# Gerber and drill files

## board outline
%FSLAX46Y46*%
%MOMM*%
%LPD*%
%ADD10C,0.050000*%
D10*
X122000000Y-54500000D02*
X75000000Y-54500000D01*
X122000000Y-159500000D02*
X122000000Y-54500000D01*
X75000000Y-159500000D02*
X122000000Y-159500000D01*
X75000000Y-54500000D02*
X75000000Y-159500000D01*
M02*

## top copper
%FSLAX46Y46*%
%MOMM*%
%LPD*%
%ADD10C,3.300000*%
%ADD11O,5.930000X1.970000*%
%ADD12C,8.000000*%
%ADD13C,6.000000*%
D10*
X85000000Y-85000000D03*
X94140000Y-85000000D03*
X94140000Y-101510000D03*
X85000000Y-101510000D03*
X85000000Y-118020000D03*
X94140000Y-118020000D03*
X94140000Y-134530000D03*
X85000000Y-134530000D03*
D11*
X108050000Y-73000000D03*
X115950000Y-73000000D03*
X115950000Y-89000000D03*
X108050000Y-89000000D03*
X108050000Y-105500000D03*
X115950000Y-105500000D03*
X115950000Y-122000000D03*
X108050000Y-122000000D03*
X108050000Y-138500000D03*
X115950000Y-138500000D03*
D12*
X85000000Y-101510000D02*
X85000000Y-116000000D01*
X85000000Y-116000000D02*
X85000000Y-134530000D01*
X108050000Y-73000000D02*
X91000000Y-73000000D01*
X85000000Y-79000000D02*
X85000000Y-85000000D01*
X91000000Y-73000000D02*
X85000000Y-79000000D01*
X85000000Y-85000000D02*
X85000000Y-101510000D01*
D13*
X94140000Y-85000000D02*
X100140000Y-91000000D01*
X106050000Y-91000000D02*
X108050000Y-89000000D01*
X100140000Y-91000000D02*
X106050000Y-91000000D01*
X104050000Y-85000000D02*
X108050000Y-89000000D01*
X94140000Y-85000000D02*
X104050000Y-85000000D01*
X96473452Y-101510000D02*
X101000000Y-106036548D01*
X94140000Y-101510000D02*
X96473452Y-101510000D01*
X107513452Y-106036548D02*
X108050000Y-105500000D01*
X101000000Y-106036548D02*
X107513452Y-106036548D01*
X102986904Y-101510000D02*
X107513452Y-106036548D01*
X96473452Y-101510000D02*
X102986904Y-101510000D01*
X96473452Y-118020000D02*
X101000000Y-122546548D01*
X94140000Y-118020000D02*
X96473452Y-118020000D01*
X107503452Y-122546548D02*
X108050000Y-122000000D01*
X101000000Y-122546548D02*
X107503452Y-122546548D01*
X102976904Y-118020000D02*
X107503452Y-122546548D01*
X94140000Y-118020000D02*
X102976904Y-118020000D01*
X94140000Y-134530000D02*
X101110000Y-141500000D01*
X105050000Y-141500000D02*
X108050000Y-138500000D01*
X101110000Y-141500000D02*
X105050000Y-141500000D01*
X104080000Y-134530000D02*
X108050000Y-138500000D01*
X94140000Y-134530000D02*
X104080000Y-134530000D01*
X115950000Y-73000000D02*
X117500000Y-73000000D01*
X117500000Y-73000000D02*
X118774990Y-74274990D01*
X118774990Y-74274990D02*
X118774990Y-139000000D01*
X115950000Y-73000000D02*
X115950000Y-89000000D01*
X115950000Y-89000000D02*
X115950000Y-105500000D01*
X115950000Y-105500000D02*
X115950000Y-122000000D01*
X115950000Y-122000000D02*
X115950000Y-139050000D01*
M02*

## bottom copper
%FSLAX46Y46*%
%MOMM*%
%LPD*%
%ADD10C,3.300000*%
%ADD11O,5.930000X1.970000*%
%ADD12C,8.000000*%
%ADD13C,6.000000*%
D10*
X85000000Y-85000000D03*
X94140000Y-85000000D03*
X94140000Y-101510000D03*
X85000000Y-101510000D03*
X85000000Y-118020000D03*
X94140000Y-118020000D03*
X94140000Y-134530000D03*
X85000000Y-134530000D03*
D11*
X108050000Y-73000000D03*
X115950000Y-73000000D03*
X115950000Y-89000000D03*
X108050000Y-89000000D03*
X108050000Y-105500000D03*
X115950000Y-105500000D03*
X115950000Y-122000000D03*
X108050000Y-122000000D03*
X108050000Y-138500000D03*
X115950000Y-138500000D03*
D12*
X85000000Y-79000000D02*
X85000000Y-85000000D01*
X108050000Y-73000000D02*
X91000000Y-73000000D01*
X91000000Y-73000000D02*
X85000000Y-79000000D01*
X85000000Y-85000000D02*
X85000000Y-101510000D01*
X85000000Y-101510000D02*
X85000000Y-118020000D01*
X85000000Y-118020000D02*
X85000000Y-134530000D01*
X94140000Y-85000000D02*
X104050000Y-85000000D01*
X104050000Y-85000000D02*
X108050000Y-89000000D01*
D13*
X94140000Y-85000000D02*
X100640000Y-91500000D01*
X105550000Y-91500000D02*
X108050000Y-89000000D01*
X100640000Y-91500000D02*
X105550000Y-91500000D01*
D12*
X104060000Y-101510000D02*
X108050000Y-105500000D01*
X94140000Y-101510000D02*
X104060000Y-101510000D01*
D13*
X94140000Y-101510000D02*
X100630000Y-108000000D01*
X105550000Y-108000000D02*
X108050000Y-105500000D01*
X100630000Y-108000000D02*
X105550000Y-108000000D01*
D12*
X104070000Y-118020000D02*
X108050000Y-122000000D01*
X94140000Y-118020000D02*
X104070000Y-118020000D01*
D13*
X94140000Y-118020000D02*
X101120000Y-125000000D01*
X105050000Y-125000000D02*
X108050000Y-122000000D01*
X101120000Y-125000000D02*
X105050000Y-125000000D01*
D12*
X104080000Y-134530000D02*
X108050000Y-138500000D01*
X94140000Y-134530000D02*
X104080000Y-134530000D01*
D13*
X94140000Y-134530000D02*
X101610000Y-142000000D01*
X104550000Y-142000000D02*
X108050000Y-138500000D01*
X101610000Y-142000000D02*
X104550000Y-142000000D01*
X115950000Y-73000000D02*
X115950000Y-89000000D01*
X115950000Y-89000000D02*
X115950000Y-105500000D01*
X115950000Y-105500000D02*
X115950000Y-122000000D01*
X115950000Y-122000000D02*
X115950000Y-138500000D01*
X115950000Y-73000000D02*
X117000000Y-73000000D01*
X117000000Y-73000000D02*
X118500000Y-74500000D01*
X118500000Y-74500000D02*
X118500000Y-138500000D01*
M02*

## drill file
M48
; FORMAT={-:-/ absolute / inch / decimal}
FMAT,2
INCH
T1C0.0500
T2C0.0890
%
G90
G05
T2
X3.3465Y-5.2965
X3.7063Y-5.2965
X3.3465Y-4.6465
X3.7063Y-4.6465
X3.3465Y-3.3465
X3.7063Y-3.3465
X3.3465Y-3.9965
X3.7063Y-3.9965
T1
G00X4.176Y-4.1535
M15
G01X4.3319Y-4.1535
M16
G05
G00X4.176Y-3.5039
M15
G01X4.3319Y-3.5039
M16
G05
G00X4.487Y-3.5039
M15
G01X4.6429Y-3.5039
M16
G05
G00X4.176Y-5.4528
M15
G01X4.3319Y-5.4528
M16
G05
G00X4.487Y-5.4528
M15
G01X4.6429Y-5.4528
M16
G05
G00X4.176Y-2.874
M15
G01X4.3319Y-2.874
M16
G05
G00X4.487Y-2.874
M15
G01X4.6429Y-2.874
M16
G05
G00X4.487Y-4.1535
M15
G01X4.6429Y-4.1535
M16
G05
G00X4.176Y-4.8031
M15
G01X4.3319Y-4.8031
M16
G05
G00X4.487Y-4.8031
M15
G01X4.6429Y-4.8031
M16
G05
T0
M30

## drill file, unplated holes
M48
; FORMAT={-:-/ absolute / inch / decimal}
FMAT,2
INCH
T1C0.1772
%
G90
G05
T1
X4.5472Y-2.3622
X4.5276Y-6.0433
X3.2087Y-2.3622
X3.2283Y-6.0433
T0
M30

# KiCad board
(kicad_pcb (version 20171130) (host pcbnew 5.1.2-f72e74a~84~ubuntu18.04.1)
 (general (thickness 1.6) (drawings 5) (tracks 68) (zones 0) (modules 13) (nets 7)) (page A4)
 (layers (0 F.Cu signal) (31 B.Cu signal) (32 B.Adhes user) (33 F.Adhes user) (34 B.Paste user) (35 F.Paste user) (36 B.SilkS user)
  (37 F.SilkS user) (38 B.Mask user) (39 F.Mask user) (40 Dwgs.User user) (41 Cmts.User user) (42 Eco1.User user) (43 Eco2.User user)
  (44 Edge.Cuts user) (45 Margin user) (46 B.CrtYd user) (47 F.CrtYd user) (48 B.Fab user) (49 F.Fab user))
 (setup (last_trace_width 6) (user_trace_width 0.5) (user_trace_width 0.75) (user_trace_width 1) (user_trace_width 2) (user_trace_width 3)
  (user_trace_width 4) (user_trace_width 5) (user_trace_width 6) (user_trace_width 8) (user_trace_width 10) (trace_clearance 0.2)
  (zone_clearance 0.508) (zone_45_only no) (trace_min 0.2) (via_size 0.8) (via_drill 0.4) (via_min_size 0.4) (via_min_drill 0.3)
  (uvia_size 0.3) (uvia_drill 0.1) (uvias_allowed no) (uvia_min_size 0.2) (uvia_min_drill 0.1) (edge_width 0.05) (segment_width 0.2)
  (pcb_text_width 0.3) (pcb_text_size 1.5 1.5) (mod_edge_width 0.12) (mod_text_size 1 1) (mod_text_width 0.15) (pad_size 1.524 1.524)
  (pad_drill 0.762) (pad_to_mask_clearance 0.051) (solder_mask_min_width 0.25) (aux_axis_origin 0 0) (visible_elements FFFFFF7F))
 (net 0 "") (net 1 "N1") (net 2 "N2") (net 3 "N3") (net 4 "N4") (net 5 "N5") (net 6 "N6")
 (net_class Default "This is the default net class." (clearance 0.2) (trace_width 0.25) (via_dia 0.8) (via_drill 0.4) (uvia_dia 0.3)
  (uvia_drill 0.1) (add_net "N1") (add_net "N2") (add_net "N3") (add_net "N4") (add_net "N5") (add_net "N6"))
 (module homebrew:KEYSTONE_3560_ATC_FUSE (layer F.Cu) (at 85 85)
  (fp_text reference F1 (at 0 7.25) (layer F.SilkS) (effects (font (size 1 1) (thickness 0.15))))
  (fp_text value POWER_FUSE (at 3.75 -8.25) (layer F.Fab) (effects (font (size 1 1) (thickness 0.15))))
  (pad 1 thru_hole circle (at 0 0) (size 3.3 3.3) (drill 2.26) (layers *.Cu *.Mask) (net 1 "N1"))
  (pad 2 thru_hole circle (at 9.14 0) (size 3.3 3.3) (drill 2.26) (layers *.Cu *.Mask) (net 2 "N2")))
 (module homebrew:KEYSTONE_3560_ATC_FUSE (layer F.Cu) (at 85 101.51)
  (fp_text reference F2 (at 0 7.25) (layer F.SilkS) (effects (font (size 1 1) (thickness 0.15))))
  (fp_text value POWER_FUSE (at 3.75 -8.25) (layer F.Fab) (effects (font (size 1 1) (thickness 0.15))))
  (pad 2 thru_hole circle (at 9.14 0) (size 3.3 3.3) (drill 2.26) (layers *.Cu *.Mask) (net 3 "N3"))
  (pad 1 thru_hole circle (at 0 0) (size 3.3 3.3) (drill 2.26) (layers *.Cu *.Mask) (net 1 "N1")))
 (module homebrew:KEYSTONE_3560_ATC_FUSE (layer F.Cu) (at 85 118.02)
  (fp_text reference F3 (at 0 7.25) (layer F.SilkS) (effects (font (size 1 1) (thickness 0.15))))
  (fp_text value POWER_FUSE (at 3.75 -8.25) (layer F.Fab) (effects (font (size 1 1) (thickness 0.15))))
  (pad 1 thru_hole circle (at 0 0) (size 3.3 3.3) (drill 2.26) (layers *.Cu *.Mask) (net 1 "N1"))
  (pad 2 thru_hole circle (at 9.14 0) (size 3.3 3.3) (drill 2.26) (layers *.Cu *.Mask) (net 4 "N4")))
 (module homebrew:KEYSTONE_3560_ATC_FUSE (layer F.Cu) (at 85 134.53)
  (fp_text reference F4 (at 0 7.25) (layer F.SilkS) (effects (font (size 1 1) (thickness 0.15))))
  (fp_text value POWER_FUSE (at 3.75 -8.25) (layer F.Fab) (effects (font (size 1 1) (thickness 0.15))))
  (pad 2 thru_hole circle (at 9.14 0) (size 3.3 3.3) (drill 2.26) (layers *.Cu *.Mask) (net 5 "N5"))
  (pad 1 thru_hole circle (at 0 0) (size 3.3 3.3) (drill 2.26) (layers *.Cu *.Mask) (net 1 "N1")))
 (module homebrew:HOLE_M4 (layer F.Cu) (at 82 153.5)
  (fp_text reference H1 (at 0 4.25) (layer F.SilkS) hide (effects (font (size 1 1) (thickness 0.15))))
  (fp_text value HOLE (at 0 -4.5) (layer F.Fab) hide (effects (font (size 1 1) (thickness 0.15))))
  (pad "" np_thru_hole circle (at 0 0) (size 4.5 4.5) (drill 4.5) (layers *.Cu *.Mask) (clearance 2.2)))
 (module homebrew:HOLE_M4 (layer F.Cu) (at 81.5 60)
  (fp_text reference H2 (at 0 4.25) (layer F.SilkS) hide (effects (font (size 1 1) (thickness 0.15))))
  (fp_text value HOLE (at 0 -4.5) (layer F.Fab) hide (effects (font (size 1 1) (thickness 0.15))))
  (pad "" np_thru_hole circle (at 0 0) (size 4.5 4.5) (drill 4.5) (layers *.Cu *.Mask) (clearance 2.2)))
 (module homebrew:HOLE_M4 (layer F.Cu) (at 115.5 60)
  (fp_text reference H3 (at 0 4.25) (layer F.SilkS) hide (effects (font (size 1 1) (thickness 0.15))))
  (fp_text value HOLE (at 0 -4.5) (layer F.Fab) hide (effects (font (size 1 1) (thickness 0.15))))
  (pad "" np_thru_hole circle (at 0 0) (size 4.5 4.5) (drill 4.5) (layers *.Cu *.Mask) (clearance 2.2)))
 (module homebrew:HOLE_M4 (layer F.Cu) (at 115 153.5)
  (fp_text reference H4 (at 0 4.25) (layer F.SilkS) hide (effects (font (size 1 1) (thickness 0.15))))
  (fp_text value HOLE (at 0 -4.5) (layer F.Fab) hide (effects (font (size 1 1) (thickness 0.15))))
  (pad "" np_thru_hole circle (at 0 0) (size 4.5 4.5) (drill 4.5) (layers *.Cu *.Mask) (clearance 2.2)))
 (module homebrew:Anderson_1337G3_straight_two (layer F.Cu) (at 112 73)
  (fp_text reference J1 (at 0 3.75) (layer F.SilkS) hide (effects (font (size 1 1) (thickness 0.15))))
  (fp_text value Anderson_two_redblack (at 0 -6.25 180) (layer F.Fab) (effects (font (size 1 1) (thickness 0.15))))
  (pad 1 thru_hole oval (at -3.95 0) (size 5.93 1.97) (drill oval 5.23 1.27) (layers *.Cu *.Mask) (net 1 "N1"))
  (pad 2 thru_hole oval (at 3.95 0) (size 5.93 1.97) (drill oval 5.23 1.27) (layers *.Cu *.Mask) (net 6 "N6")))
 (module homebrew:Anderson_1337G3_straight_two (layer F.Cu) (at 112 89)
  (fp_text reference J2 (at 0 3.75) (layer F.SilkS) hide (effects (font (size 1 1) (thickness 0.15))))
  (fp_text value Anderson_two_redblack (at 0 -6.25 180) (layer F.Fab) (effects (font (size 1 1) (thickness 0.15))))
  (pad 2 thru_hole oval (at 3.95 0) (size 5.93 1.97) (drill oval 5.23 1.27) (layers *.Cu *.Mask) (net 6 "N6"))
  (pad 1 thru_hole oval (at -3.95 0) (size 5.93 1.97) (drill oval 5.23 1.27) (layers *.Cu *.Mask) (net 2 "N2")))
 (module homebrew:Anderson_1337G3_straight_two (layer F.Cu) (at 112 105.5)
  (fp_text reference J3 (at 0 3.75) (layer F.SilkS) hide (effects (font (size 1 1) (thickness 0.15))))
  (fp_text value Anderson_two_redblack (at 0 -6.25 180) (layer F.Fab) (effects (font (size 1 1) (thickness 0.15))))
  (pad 1 thru_hole oval (at -3.95 0) (size 5.93 1.97) (drill oval 5.23 1.27) (layers *.Cu *.Mask) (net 3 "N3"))
  (pad 2 thru_hole oval (at 3.95 0) (size 5.93 1.97) (drill oval 5.23 1.27) (layers *.Cu *.Mask) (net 6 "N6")))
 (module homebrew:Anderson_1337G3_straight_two (layer F.Cu) (at 112 122)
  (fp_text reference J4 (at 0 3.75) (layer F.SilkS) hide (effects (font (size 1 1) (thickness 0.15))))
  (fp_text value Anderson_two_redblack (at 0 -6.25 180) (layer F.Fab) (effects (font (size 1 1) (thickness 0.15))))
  (pad 2 thru_hole oval (at 3.95 0) (size 5.93 1.97) (drill oval 5.23 1.27) (layers *.Cu *.Mask) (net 6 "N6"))
  (pad 1 thru_hole oval (at -3.95 0) (size 5.93 1.97) (drill oval 5.23 1.27) (layers *.Cu *.Mask) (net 4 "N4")))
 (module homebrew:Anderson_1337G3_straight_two (layer F.Cu) (at 112 138.5)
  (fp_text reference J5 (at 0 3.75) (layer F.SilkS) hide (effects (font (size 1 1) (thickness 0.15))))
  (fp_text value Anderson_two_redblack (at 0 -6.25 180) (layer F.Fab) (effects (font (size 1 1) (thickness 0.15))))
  (pad 1 thru_hole oval (at -3.95 0) (size 5.93 1.97) (drill oval 5.23 1.27) (layers *.Cu *.Mask) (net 5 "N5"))
  (pad 2 thru_hole oval (at 3.95 0) (size 5.93 1.97) (drill oval 5.23 1.27) (layers *.Cu *.Mask) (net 6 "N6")))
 (gr_line (start 122 54.5) (end 75 54.5) (layer Edge.Cuts) (width 0.05))
 (gr_line (start 122 159.5) (end 122 54.5) (layer Edge.Cuts) (width 0.05))
 (gr_line (start 75 159.5) (end 122 159.5) (layer Edge.Cuts) (width 0.05))
 (gr_line (start 75 54.5) (end 75 159.5) (layer Edge.Cuts) (width 0.05))
 (segment (start 85 101.51) (end 85 116) (width 8) (layer F.Cu) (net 1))
 (segment (start 85 116) (end 85 134.53) (width 8) (layer F.Cu) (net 1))
 (segment (start 85 79) (end 85 85) (width 8) (layer B.Cu) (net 1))
 (segment (start 108.05 73) (end 91 73) (width 8) (layer B.Cu) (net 1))
 (segment (start 91 73) (end 85 79) (width 8) (layer B.Cu) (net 1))
 (segment (start 85 85) (end 85 101.51) (width 8) (layer B.Cu) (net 1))
 (segment (start 85 101.51) (end 85 118.02) (width 8) (layer B.Cu) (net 1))
 (segment (start 85 118.02) (end 85 134.53) (width 8) (layer B.Cu) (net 1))
 (segment (start 108.05 73) (end 91 73) (width 8) (layer F.Cu) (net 1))
 (segment (start 85 79) (end 85 85) (width 8) (layer F.Cu) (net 1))
 (segment (start 91 73) (end 85 79) (width 8) (layer F.Cu) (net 1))
 (segment (start 85 85) (end 85 101.51) (width 8) (layer F.Cu) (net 1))
 (segment (start 94.14 85) (end 104.05 85) (width 8) (layer B.Cu) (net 2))
 (segment (start 104.05 85) (end 108.05 89) (width 8) (layer B.Cu) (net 2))
 (segment (start 94.14 85) (end 100.64 91.5) (width 6) (layer B.Cu) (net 2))
 (segment (start 105.55 91.5) (end 108.05 89) (width 6) (layer B.Cu) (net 2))
 (segment (start 100.64 91.5) (end 105.55 91.5) (width 6) (layer B.Cu) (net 2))
 (segment (start 94.14 85) (end 100.14 91) (width 6) (layer F.Cu) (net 2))
 (segment (start 106.05 91) (end 108.05 89) (width 6) (layer F.Cu) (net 2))
 (segment (start 100.14 91) (end 106.05 91) (width 6) (layer F.Cu) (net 2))
 (segment (start 104.05 85) (end 108.05 89) (width 6) (layer F.Cu) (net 2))
 (segment (start 94.14 85) (end 104.05 85) (width 6) (layer F.Cu) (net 2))
 (segment (start 104.06 101.51) (end 108.05 105.5) (width 8) (layer B.Cu) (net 3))
 (segment (start 94.14 101.51) (end 104.06 101.51) (width 8) (layer B.Cu) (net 3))
 (segment (start 94.14 101.51) (end 100.63 108) (width 6) (layer B.Cu) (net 3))
 (segment (start 105.55 108) (end 108.05 105.5) (width 6) (layer B.Cu) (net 3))
 (segment (start 100.63 108) (end 105.55 108) (width 6) (layer B.Cu) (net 3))
 (segment (start 96.473452 101.51) (end 101 106.036548) (width 6) (layer F.Cu) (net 3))
 (segment (start 94.14 101.51) (end 96.473452 101.51) (width 6) (layer F.Cu) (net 3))
 (segment (start 107.513452 106.036548) (end 108.05 105.5) (width 6) (layer F.Cu) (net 3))
 (segment (start 101 106.036548) (end 107.513452 106.036548) (width 6) (layer F.Cu) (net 3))
 (segment (start 102.986904 101.51) (end 107.513452 106.036548) (width 6) (layer F.Cu) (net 3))
 (segment (start 96.473452 101.51) (end 102.986904 101.51) (width 6) (layer F.Cu) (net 3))
 (segment (start 104.07 118.02) (end 108.05 122) (width 8) (layer B.Cu) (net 4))
 (segment (start 94.14 118.02) (end 104.07 118.02) (width 8) (layer B.Cu) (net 4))
 (segment (start 94.14 118.02) (end 101.12 125) (width 6) (layer B.Cu) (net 4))
 (segment (start 105.05 125) (end 108.05 122) (width 6) (layer B.Cu) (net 4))
 (segment (start 101.12 125) (end 105.05 125) (width 6) (layer B.Cu) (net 4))
 (segment (start 96.473452 118.02) (end 101 122.546548) (width 6) (layer F.Cu) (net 4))
 (segment (start 94.14 118.02) (end 96.473452 118.02) (width 6) (layer F.Cu) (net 4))
 (segment (start 107.503452 122.546548) (end 108.05 122) (width 6) (layer F.Cu) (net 4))
 (segment (start 101 122.546548) (end 107.503452 122.546548) (width 6) (layer F.Cu) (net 4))
 (segment (start 102.976904 118.02) (end 107.503452 122.546548) (width 6) (layer F.Cu) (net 4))
 (segment (start 94.14 118.02) (end 102.976904 118.02) (width 6) (layer F.Cu) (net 4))
 (segment (start 104.08 134.53) (end 108.05 138.5) (width 8) (layer B.Cu) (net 5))
 (segment (start 94.14 134.53) (end 104.08 134.53) (width 8) (layer B.Cu) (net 5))
 (segment (start 94.14 134.53) (end 101.61 142) (width 6) (layer B.Cu) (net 5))
 (segment (start 104.55 142) (end 108.05 138.5) (width 6) (layer B.Cu) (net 5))
 (segment (start 101.61 142) (end 104.55 142) (width 6) (layer B.Cu) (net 5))
 (segment (start 94.14 134.53) (end 101.11 141.5) (width 6) (layer F.Cu) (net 5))
 (segment (start 105.05 141.5) (end 108.05 138.5) (width 6) (layer F.Cu) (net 5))
 (segment (start 101.11 141.5) (end 105.05 141.5) (width 6) (layer F.Cu) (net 5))
 (segment (start 104.08 134.53) (end 108.05 138.5) (width 6) (layer F.Cu) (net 5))
 (segment (start 94.14 134.53) (end 104.08 134.53) (width 6) (layer F.Cu) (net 5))
 (segment (start 115.95 73) (end 115.95 89) (width 6) (layer B.Cu) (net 6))
 (segment (start 115.95 89) (end 115.95 105.5) (width 6) (layer B.Cu) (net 6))
 (segment (start 115.95 105.5) (end 115.95 122) (width 6) (layer B.Cu) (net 6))
 (segment (start 115.95 122) (end 115.95 138.5) (width 6) (layer B.Cu) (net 6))
 (segment (start 115.95 73) (end 117 73) (width 6) (layer B.Cu) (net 6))
 (segment (start 117 73) (end 118.5 74.5) (width 6) (layer B.Cu) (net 6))
 (segment (start 118.5 74.5) (end 118.5 138.5) (width 6) (layer B.Cu) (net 6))
 (segment (start 115.95 73) (end 117.5 73) (width 6) (layer F.Cu) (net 6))
 (segment (start 117.5 73) (end 118.77499 74.27499) (width 6) (layer F.Cu) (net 6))
 (segment (start 118.77499 74.27499) (end 118.77499 139) (width 6) (layer F.Cu) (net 6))
 (segment (start 115.95 73) (end 115.95 89) (width 6) (layer F.Cu) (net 6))
 (segment (start 115.95 89) (end 115.95 105.5) (width 6) (layer F.Cu) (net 6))
 (segment (start 115.95 105.5) (end 115.95 122) (width 6) (layer F.Cu) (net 6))
 (segment (start 115.95 122) (end 115.95 139.05) (width 6) (layer F.Cu) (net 6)))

